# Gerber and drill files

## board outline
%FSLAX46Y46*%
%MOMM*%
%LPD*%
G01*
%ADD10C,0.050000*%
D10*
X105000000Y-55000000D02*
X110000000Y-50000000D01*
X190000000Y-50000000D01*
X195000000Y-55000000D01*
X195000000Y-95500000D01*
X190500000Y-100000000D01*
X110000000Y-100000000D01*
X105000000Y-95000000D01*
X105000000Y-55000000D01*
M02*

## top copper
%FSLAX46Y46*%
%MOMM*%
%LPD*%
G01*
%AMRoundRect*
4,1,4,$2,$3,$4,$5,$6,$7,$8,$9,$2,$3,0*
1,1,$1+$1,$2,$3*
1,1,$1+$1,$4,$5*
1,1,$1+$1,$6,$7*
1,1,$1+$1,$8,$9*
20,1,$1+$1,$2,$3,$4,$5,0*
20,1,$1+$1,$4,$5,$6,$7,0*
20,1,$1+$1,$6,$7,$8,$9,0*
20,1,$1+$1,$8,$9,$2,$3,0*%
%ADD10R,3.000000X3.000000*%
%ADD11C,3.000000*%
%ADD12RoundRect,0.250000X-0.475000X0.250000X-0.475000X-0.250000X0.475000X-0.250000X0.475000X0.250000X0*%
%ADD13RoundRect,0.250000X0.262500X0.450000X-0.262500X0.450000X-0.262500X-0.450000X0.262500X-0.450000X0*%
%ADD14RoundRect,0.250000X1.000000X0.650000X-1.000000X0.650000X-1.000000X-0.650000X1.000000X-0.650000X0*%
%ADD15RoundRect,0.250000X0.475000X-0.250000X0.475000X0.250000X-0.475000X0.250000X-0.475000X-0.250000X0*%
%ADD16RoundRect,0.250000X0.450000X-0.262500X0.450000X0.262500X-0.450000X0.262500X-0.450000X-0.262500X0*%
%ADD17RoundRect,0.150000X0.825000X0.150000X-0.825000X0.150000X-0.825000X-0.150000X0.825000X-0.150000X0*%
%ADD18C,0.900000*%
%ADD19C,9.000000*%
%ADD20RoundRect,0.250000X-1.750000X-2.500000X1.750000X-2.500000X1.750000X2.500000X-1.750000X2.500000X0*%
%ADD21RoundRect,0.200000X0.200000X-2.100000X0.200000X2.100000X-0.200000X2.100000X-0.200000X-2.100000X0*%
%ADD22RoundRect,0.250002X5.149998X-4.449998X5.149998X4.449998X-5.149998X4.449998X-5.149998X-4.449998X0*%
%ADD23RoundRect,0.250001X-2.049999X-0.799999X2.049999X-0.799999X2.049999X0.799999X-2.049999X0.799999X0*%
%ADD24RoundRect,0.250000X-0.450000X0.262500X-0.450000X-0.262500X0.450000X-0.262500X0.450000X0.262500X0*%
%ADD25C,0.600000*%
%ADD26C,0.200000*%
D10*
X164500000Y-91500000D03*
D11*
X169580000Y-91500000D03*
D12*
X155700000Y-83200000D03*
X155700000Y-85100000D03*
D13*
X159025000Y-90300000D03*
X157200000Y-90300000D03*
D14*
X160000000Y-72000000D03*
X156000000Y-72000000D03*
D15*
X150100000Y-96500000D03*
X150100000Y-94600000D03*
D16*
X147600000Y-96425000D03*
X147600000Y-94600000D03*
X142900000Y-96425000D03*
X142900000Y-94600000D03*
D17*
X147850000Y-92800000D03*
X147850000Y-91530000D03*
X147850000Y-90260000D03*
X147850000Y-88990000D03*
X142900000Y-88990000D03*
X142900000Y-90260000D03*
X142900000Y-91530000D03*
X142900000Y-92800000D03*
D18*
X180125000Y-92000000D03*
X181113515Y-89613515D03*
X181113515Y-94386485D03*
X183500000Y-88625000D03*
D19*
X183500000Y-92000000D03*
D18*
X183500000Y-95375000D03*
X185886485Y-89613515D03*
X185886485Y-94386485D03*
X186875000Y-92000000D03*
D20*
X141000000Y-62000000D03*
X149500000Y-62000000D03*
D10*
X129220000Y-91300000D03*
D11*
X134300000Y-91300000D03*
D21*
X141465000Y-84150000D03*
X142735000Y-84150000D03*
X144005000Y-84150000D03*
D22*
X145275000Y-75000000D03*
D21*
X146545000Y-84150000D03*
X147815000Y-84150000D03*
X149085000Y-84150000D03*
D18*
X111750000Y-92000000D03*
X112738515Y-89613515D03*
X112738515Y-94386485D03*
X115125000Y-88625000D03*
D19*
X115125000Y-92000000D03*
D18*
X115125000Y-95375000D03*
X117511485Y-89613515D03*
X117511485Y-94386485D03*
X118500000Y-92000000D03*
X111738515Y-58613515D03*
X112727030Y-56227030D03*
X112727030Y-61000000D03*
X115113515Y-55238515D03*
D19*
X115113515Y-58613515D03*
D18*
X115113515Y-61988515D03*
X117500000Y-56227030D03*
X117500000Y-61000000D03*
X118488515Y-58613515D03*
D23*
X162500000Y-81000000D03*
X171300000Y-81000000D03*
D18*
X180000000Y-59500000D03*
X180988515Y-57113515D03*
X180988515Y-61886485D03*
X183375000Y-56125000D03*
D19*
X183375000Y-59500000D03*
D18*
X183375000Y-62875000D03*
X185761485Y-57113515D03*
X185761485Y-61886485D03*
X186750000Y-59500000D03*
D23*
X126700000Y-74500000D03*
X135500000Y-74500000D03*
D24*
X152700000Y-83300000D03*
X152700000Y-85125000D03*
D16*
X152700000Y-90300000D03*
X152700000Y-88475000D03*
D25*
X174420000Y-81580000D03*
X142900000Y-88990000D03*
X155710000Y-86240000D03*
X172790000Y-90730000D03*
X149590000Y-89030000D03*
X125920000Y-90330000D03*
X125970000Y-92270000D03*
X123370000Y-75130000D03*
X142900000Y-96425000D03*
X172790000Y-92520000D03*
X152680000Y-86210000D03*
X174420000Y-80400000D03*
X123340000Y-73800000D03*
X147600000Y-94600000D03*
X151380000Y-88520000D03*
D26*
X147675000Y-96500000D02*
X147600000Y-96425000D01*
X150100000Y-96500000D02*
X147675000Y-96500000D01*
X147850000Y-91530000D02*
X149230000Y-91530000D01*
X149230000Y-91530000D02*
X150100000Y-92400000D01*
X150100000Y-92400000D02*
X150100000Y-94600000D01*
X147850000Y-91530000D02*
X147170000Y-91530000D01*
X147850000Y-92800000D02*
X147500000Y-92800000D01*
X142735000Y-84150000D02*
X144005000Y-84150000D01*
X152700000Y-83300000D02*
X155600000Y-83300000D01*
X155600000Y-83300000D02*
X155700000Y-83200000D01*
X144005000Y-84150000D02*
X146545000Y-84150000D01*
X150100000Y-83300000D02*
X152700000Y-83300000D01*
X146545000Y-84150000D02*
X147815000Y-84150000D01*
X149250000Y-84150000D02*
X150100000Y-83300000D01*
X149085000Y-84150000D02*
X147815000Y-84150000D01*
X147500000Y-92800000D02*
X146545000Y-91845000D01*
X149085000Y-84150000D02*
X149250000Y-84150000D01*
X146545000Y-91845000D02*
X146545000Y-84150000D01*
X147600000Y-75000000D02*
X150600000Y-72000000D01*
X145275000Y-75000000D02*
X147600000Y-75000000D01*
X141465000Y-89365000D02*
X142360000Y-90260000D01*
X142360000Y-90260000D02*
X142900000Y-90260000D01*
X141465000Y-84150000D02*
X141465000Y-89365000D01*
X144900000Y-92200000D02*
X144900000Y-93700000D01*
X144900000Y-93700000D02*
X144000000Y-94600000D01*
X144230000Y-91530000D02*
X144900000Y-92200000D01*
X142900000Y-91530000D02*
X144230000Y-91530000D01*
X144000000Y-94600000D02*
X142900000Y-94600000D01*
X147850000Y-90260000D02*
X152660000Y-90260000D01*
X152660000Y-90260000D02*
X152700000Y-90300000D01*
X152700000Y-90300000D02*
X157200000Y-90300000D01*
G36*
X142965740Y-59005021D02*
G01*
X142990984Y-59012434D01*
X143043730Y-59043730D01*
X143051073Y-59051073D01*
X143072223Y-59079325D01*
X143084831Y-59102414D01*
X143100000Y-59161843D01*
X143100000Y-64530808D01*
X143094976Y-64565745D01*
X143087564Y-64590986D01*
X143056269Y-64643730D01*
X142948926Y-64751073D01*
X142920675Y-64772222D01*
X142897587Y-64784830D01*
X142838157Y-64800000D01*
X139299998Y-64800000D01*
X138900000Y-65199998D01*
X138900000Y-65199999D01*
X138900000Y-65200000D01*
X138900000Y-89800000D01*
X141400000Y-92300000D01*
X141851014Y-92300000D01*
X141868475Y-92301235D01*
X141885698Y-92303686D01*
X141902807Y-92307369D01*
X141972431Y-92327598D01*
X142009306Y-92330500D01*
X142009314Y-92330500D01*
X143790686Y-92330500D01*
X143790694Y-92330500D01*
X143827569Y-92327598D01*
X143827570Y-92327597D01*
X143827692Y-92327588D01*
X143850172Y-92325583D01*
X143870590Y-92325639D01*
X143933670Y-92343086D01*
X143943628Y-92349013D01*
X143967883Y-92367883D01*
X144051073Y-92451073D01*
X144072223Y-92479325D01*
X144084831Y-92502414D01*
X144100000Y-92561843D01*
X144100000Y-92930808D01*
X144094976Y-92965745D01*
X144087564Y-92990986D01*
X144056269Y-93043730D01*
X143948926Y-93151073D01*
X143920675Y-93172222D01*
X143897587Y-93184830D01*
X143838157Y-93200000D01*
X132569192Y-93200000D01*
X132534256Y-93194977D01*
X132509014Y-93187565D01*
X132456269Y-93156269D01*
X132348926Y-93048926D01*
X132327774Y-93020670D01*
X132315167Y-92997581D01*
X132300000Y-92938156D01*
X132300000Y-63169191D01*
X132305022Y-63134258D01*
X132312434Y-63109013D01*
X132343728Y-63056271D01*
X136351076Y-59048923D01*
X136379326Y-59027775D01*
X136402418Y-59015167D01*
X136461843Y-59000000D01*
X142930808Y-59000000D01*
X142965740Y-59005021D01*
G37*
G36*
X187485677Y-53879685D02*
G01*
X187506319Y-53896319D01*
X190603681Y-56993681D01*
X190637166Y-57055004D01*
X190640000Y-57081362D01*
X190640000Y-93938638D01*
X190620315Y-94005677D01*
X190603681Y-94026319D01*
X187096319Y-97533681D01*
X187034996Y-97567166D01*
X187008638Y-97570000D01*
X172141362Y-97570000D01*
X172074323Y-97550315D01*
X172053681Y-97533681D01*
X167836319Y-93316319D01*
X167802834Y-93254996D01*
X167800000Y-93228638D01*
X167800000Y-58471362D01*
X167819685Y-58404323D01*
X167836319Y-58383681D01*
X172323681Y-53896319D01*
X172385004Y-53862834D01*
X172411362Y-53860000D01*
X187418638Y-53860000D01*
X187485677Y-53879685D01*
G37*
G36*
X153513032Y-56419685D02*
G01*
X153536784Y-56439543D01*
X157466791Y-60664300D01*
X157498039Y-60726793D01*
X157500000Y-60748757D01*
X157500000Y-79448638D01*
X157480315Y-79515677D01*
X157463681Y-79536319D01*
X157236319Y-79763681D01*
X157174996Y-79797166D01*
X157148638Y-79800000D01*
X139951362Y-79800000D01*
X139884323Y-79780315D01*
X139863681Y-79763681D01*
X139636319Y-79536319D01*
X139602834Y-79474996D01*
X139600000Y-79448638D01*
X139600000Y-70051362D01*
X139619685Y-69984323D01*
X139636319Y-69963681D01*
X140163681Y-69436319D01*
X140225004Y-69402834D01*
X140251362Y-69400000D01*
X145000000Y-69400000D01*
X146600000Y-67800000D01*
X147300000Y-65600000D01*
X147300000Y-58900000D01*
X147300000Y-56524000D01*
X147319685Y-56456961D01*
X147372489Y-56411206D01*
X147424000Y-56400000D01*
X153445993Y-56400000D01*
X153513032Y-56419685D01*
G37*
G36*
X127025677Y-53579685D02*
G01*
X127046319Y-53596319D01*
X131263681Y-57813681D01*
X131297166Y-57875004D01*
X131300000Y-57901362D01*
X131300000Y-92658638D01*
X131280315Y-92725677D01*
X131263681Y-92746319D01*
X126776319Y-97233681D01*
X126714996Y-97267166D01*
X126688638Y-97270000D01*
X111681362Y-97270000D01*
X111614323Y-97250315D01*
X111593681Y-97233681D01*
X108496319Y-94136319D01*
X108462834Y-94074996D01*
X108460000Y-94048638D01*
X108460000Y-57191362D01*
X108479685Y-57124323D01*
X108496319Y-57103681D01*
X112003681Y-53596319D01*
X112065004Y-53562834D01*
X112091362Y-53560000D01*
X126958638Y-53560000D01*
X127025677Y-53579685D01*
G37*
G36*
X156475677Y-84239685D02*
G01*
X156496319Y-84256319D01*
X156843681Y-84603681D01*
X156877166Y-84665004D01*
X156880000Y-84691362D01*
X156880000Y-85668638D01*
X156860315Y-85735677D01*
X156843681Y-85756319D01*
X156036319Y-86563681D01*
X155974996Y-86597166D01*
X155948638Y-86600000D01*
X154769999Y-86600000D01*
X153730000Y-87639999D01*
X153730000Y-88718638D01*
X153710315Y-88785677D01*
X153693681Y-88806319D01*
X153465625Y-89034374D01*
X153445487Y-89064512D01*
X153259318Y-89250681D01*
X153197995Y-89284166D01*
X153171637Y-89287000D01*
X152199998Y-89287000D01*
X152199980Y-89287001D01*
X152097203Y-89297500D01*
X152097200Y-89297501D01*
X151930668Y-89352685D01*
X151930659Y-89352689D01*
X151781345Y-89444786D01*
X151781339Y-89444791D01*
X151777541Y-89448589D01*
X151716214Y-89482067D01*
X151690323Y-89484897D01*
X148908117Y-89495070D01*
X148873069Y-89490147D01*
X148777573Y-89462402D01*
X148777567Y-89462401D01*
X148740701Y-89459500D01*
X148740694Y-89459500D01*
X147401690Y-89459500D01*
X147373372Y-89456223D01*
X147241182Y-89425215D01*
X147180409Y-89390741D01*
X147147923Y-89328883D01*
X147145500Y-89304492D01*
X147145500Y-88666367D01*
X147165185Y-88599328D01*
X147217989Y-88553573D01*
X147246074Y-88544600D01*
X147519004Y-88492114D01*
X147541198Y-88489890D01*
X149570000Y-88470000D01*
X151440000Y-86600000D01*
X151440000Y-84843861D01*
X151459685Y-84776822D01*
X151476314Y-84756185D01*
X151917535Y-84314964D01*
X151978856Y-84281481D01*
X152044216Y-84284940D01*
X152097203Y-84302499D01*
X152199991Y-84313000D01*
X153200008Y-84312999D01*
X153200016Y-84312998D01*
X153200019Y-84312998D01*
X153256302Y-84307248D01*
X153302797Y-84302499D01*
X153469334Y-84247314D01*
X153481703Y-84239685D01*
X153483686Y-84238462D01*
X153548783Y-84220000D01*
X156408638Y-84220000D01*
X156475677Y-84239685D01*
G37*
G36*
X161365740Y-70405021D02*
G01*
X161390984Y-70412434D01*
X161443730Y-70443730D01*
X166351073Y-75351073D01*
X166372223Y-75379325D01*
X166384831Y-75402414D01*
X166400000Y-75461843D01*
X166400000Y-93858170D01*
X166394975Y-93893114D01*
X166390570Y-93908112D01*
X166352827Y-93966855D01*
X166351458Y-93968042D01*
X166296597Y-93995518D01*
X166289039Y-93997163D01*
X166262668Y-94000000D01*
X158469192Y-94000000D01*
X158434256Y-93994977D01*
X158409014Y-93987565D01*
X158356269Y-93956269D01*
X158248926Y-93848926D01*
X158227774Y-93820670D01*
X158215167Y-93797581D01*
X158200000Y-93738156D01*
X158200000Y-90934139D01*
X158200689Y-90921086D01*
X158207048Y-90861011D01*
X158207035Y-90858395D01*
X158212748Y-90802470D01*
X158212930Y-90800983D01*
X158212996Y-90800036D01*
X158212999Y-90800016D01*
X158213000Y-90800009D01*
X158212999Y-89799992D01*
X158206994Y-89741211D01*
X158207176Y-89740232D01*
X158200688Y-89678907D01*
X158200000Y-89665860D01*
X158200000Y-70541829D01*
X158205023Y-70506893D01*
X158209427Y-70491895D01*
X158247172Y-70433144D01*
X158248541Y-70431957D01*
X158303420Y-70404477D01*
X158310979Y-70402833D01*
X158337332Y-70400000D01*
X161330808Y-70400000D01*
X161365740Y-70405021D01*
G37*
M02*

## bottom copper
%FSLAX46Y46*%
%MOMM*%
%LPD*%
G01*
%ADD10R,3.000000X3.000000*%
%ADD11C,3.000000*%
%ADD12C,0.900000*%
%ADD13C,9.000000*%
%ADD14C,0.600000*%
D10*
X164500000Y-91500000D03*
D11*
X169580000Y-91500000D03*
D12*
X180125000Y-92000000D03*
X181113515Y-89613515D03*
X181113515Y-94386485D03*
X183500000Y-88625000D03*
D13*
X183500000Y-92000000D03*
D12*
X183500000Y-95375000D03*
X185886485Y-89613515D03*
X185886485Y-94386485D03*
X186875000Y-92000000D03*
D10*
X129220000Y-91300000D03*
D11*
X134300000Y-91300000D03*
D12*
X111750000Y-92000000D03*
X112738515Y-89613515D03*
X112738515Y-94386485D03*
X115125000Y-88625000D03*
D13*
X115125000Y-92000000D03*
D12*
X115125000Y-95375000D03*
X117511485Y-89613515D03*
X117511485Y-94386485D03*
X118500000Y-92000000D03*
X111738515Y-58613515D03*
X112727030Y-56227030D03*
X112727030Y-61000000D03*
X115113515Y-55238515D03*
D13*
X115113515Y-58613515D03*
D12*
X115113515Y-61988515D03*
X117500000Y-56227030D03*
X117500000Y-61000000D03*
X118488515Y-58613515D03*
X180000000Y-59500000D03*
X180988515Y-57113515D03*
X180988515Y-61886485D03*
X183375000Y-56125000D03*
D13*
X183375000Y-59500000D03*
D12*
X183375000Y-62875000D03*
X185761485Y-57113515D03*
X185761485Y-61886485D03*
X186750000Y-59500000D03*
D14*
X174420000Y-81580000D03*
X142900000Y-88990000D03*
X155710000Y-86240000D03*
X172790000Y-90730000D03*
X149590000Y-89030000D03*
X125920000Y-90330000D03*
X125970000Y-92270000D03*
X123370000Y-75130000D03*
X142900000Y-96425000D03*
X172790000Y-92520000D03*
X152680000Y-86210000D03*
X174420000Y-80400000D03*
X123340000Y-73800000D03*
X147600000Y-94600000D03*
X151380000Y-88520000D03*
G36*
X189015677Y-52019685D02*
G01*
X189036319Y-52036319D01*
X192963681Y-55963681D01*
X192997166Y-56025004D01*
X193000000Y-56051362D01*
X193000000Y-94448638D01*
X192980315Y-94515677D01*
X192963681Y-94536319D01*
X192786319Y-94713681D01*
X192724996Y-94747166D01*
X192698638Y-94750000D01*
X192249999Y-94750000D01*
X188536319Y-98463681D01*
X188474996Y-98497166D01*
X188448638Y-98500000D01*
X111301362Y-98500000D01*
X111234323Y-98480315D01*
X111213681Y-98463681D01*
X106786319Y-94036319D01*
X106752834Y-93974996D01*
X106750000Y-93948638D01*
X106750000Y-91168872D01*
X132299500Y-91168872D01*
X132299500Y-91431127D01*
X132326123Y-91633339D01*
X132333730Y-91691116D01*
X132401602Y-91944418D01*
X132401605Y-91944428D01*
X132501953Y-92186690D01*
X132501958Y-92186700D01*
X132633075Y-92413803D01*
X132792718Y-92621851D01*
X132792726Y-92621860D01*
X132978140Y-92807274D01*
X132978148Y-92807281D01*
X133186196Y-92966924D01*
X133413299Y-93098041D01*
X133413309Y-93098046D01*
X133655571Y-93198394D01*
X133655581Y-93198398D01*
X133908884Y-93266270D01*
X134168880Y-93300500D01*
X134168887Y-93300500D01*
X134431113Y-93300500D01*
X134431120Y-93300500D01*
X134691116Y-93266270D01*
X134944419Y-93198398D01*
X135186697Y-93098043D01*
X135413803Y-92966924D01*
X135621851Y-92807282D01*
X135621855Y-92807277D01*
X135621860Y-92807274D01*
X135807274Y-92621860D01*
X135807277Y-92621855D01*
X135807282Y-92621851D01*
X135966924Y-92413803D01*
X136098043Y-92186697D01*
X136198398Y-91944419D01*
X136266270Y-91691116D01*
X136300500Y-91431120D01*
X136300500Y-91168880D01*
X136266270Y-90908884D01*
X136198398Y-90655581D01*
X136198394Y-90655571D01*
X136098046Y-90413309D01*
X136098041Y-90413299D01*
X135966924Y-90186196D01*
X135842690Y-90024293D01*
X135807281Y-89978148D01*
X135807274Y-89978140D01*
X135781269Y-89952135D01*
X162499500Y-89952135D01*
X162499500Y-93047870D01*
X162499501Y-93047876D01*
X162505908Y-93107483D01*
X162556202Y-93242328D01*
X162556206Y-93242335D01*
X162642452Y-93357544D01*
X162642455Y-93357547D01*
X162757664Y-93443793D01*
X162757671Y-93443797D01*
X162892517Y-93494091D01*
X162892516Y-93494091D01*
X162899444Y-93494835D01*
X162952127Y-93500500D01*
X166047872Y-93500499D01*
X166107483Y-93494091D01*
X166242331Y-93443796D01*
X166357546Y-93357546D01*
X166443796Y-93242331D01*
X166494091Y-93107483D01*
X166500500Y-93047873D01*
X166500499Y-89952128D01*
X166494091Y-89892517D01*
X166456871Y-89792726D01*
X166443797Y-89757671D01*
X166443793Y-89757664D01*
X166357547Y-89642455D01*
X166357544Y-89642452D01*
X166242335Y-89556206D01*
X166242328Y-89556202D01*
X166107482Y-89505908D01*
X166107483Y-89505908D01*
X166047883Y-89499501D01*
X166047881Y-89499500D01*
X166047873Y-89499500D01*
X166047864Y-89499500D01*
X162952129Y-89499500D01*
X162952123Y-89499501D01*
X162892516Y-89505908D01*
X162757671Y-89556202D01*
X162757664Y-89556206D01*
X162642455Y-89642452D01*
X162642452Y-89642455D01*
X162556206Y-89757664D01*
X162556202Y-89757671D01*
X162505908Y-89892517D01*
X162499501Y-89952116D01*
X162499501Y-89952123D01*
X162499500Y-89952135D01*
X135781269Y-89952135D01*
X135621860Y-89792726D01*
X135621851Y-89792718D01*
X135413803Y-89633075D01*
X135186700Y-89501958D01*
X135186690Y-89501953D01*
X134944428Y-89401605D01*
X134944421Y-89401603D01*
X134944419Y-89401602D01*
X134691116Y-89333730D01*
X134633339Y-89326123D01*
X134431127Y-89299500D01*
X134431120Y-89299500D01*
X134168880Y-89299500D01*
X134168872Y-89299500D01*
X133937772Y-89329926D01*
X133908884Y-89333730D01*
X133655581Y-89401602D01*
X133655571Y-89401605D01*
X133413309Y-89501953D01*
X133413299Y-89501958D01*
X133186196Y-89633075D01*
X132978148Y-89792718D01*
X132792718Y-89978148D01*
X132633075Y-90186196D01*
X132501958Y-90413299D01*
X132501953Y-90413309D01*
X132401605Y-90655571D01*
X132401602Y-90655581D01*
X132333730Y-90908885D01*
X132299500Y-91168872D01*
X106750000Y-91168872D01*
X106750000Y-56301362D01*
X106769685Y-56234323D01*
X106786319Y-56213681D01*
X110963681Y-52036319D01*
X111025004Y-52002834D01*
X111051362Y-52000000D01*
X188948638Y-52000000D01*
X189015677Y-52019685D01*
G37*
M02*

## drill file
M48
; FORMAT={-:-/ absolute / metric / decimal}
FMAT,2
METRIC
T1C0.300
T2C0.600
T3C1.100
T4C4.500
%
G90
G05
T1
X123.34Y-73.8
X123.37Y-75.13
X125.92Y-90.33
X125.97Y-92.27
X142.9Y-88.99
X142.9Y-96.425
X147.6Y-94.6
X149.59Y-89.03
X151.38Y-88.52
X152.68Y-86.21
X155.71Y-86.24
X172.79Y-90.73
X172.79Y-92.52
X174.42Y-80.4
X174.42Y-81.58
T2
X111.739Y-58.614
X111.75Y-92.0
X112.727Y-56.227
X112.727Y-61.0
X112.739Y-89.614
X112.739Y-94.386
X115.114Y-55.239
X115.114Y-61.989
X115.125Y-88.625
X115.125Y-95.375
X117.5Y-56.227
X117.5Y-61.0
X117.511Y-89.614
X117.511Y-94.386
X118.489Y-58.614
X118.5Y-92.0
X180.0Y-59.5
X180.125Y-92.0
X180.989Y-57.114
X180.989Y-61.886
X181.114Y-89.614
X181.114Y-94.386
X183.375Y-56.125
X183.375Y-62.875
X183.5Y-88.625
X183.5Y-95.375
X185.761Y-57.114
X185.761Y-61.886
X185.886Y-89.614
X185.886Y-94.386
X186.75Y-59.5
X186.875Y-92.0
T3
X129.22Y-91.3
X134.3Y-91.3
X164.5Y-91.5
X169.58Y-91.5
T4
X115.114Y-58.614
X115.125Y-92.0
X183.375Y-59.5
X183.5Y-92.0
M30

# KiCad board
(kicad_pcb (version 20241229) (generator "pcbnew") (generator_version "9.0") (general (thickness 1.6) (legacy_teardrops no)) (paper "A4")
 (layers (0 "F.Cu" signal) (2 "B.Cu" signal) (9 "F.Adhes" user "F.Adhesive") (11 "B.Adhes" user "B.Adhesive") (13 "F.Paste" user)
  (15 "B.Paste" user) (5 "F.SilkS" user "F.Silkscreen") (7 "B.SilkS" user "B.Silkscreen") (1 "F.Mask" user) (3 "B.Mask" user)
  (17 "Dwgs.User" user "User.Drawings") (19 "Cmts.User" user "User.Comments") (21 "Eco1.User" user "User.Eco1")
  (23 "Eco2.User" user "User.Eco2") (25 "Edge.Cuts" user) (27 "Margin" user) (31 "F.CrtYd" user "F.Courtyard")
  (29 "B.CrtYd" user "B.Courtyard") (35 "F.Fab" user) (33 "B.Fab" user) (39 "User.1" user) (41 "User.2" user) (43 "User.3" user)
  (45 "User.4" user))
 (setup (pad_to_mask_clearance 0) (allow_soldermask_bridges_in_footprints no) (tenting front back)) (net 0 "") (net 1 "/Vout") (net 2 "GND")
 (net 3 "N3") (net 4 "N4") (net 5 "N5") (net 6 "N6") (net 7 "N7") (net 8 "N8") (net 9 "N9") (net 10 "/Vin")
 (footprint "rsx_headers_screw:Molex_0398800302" (layer "F.Cu") (at 164.5 91.5)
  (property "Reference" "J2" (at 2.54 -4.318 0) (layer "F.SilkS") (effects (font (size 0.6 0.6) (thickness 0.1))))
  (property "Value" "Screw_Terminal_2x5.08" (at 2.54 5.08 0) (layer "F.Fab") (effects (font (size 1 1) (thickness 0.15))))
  (pad "1" thru_hole rect (at 0 0) (size 3 3) (drill 1.1) (layers "*.Cu" "*.Mask") (remove_unused_layers no) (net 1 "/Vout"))
  (pad "2" thru_hole circle (at 5.08 0) (size 3 3) (drill 1.1) (layers "*.Cu" "*.Mask") (remove_unused_layers no) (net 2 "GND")))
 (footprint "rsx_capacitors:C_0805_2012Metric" (layer "F.Cu") (at 155.7 84.15 -90)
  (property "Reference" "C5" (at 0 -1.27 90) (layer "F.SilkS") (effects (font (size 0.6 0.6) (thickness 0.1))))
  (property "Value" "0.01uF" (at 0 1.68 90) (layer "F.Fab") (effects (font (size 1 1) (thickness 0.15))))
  (pad "1" smd roundrect (at -0.95 0 270) (size 1 1.45) (layers "F.Cu" "F.Mask" "F.Paste") (roundrect_rratio 0.25) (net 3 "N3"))
  (pad "2" smd roundrect (at 0.95 0 270) (size 1 1.45) (layers "F.Cu" "F.Mask" "F.Paste") (roundrect_rratio 0.25) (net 2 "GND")))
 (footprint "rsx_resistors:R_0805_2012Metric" (layer "F.Cu") (at 158.1125 90.3 180)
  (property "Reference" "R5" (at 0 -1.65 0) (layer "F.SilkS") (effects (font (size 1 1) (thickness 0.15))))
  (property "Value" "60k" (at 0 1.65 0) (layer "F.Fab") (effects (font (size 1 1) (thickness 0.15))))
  (pad "1" smd roundrect (at -0.9125 0 180) (size 1.025 1.4) (layers "F.Cu" "F.Mask" "F.Paste") (roundrect_rratio 0.243902) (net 1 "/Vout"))
  (pad "2" smd roundrect (at 0.9125 0 180) (size 1.025 1.4) (layers "F.Cu" "F.Mask" "F.Paste") (roundrect_rratio 0.243902) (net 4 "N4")))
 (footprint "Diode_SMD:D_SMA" (layer "F.Cu") (at 158 72 180)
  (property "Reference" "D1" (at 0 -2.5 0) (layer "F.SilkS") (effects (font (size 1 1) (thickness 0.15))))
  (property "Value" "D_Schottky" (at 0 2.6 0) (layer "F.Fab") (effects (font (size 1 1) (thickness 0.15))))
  (pad "1" smd roundrect (at -2 0 180) (size 2.5 1.8) (layers "F.Cu" "F.Mask" "F.Paste") (roundrect_rratio 0.1388888889) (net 1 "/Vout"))
  (pad "2" smd roundrect (at 2 0 180) (size 2.5 1.8) (layers "F.Cu" "F.Mask" "F.Paste") (roundrect_rratio 0.1388888889) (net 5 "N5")))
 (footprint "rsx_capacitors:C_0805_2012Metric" (layer "F.Cu") (at 150.1 95.55 90)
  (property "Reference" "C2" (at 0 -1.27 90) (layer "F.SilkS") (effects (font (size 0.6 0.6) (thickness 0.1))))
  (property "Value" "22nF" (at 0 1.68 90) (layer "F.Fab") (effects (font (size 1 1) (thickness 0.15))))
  (pad "1" smd roundrect (at -0.95 0 90) (size 1 1.45) (layers "F.Cu" "F.Mask" "F.Paste") (roundrect_rratio 0.25) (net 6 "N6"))
  (pad "2" smd roundrect (at 0.95 0 90) (size 1 1.45) (layers "F.Cu" "F.Mask" "F.Paste") (roundrect_rratio 0.25) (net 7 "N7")))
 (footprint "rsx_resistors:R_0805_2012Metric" (layer "F.Cu") (at 147.6 95.5125 90)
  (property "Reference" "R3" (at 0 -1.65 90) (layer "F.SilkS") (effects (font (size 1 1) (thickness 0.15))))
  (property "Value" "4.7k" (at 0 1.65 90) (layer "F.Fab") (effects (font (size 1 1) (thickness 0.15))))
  (pad "1" smd roundrect (at -0.9125 0 90) (size 1.025 1.4) (layers "F.Cu" "F.Mask" "F.Paste") (roundrect_rratio 0.243902) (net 6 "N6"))
  (pad "2" smd roundrect (at 0.9125 0 90) (size 1.025 1.4) (layers "F.Cu" "F.Mask" "F.Paste") (roundrect_rratio 0.243902) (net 2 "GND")))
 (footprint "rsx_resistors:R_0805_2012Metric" (layer "F.Cu") (at 142.9 95.5125 90)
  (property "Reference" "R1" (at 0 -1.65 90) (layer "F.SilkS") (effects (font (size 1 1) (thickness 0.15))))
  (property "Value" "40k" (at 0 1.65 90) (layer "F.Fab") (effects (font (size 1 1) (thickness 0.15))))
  (pad "1" smd roundrect (at -0.9125 0 90) (size 1.025 1.4) (layers "F.Cu" "F.Mask" "F.Paste") (roundrect_rratio 0.243902) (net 2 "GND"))
  (pad "2" smd roundrect (at 0.9125 0 90) (size 1.025 1.4) (layers "F.Cu" "F.Mask" "F.Paste") (roundrect_rratio 0.243902) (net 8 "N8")))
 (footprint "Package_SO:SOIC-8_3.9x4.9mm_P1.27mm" (layer "F.Cu") (at 145.375 90.895 180)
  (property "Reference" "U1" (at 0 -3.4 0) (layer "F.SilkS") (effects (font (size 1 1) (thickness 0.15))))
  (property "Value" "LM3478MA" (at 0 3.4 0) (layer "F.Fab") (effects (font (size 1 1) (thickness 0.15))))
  (pad "1" smd roundrect (at -2.475 -1.905 180) (size 1.95 0.6) (layers "F.Cu" "F.Mask" "F.Paste") (roundrect_rratio 0.25) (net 3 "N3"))
  (pad "2" smd roundrect (at -2.475 -0.635 180) (size 1.95 0.6) (layers "F.Cu" "F.Mask" "F.Paste") (roundrect_rratio 0.25) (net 7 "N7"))
  (pad "3" smd roundrect (at -2.475 0.635 180) (size 1.95 0.6) (layers "F.Cu" "F.Mask" "F.Paste") (roundrect_rratio 0.25) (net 4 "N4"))
  (pad "4" smd roundrect (at -2.475 1.905 180) (size 1.95 0.6) (layers "F.Cu" "F.Mask" "F.Paste") (roundrect_rratio 0.25) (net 2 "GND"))
  (pad "5" smd roundrect (at 2.475 1.905 180) (size 1.95 0.6) (layers "F.Cu" "F.Mask" "F.Paste") (roundrect_rratio 0.25) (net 2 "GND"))
  (pad "6" smd roundrect (at 2.475 0.635 180) (size 1.95 0.6) (layers "F.Cu" "F.Mask" "F.Paste") (roundrect_rratio 0.25) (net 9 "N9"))
  (pad "7" smd roundrect (at 2.475 -0.635 180) (size 1.95 0.6) (layers "F.Cu" "F.Mask" "F.Paste") (roundrect_rratio 0.25) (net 8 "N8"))
  (pad "8" smd roundrect (at 2.475 -1.905 180) (size 1.95 0.6) (layers "F.Cu" "F.Mask" "F.Paste") (roundrect_rratio 0.25) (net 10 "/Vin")))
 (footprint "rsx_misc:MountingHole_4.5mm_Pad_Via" (layer "F.Cu") (at 183.5 92)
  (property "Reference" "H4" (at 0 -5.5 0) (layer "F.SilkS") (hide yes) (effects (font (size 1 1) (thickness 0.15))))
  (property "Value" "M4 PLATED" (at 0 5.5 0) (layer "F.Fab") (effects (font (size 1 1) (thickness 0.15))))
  (pad "1" thru_hole circle (at -3.375 0) (size 0.9 0.9) (drill 0.6) (layers "*.Cu" "*.Mask") (remove_unused_layers no) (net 2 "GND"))
  (pad "1" thru_hole circle (at -2.386485 -2.386485) (size 0.9 0.9) (drill 0.6) (layers "*.Cu" "*.Mask") (remove_unused_layers no)
   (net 2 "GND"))
  (pad "1" thru_hole circle (at -2.386485 2.386485) (size 0.9 0.9) (drill 0.6) (layers "*.Cu" "*.Mask") (remove_unused_layers no)
   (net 2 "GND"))
  (pad "1" thru_hole circle (at 0 -3.375) (size 0.9 0.9) (drill 0.6) (layers "*.Cu" "*.Mask") (remove_unused_layers no) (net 2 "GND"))
  (pad "1" thru_hole circle (at 0 0) (size 9 9) (drill 4.5) (layers "*.Cu" "*.Mask") (remove_unused_layers no) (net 2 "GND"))
  (pad "1" thru_hole circle (at 0 3.375) (size 0.9 0.9) (drill 0.6) (layers "*.Cu" "*.Mask") (remove_unused_layers no) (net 2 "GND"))
  (pad "1" thru_hole circle (at 2.386485 -2.386485) (size 0.9 0.9) (drill 0.6) (layers "*.Cu" "*.Mask") (remove_unused_layers no)
   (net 2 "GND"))
  (pad "1" thru_hole circle (at 2.386485 2.386485) (size 0.9 0.9) (drill 0.6) (layers "*.Cu" "*.Mask") (remove_unused_layers no)
   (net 2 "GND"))
  (pad "1" thru_hole circle (at 3.375 0) (size 0.9 0.9) (drill 0.6) (layers "*.Cu" "*.Mask") (remove_unused_layers no) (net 2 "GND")))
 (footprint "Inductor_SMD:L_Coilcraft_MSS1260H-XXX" (layer "F.Cu") (at 145.25 62)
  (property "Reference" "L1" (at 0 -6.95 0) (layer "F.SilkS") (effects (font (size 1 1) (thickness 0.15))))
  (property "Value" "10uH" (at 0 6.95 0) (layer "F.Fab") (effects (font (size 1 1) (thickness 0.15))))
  (pad "1" smd roundrect (at -4.25 0) (size 4 5.5) (layers "F.Cu" "F.Mask" "F.Paste") (roundrect_rratio 0.0625) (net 10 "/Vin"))
  (pad "2" smd roundrect (at 4.25 0) (size 4 5.5) (layers "F.Cu" "F.Mask" "F.Paste") (roundrect_rratio 0.0625) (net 5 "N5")))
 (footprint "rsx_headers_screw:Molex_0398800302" (layer "F.Cu") (at 129.22 91.3)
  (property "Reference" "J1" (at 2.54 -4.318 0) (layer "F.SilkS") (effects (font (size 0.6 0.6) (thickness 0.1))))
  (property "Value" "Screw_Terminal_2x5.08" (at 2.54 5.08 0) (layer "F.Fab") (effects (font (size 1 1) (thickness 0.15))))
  (pad "1" thru_hole rect (at 0 0) (size 3 3) (drill 1.1) (layers "*.Cu" "*.Mask") (remove_unused_layers no) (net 2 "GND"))
  (pad "2" thru_hole circle (at 5.08 0) (size 3 3) (drill 1.1) (layers "*.Cu" "*.Mask") (remove_unused_layers no) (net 10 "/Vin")))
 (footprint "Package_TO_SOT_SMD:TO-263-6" (layer "F.Cu") (at 145.275 76.5 90)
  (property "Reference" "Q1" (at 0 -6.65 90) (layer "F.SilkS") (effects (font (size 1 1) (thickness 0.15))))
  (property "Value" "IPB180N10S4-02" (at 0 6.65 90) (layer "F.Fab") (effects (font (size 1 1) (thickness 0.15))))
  (pad "" smd roundrect (at -0.925 -2.775 90) (size 4.55 5.25) (layers "F.Paste") (roundrect_rratio 0.054945))
  (pad "" smd roundrect (at -0.925 2.775 90) (size 4.55 5.25) (layers "F.Paste") (roundrect_rratio 0.054945))
  (pad "" smd roundrect (at 3.925 -2.775 90) (size 4.55 5.25) (layers "F.Paste") (roundrect_rratio 0.054945))
  (pad "" smd roundrect (at 3.925 2.775 90) (size 4.55 5.25) (layers "F.Paste") (roundrect_rratio 0.054945))
  (pad "1" smd roundrect (at -7.65 -3.81 90) (size 4.6 0.8) (layers "F.Cu" "F.Mask" "F.Paste") (roundrect_rratio 0.25) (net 9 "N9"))
  (pad "2" smd roundrect (at -7.65 -2.54 90) (size 4.6 0.8) (layers "F.Cu" "F.Mask" "F.Paste") (roundrect_rratio 0.25) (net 3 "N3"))
  (pad "3" smd roundrect (at -7.65 -1.27 90) (size 4.6 0.8) (layers "F.Cu" "F.Mask" "F.Paste") (roundrect_rratio 0.25) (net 3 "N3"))
  (pad "4" smd roundrect (at 1.5 0 90) (size 9.4 10.8) (layers "F.Cu" "F.Mask") (roundrect_rratio 0.026596) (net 5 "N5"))
  (pad "5" smd roundrect (at -7.65 1.27 90) (size 4.6 0.8) (layers "F.Cu" "F.Mask" "F.Paste") (roundrect_rratio 0.25) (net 3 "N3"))
  (pad "6" smd roundrect (at -7.65 2.54 90) (size 4.6 0.8) (layers "F.Cu" "F.Mask" "F.Paste") (roundrect_rratio 0.25) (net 3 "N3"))
  (pad "7" smd roundrect (at -7.65 3.81 90) (size 4.6 0.8) (layers "F.Cu" "F.Mask" "F.Paste") (roundrect_rratio 0.25) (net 3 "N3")))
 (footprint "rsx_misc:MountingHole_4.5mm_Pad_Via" (layer "F.Cu") (at 115.125 92)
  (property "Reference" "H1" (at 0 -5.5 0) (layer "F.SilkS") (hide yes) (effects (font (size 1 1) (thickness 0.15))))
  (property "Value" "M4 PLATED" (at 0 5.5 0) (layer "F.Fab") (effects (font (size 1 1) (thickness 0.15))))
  (pad "1" thru_hole circle (at -3.375 0) (size 0.9 0.9) (drill 0.6) (layers "*.Cu" "*.Mask") (remove_unused_layers no) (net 2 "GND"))
  (pad "1" thru_hole circle (at -2.386485 -2.386485) (size 0.9 0.9) (drill 0.6) (layers "*.Cu" "*.Mask") (remove_unused_layers no)
   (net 2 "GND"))
  (pad "1" thru_hole circle (at -2.386485 2.386485) (size 0.9 0.9) (drill 0.6) (layers "*.Cu" "*.Mask") (remove_unused_layers no)
   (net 2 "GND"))
  (pad "1" thru_hole circle (at 0 -3.375) (size 0.9 0.9) (drill 0.6) (layers "*.Cu" "*.Mask") (remove_unused_layers no) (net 2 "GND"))
  (pad "1" thru_hole circle (at 0 0) (size 9 9) (drill 4.5) (layers "*.Cu" "*.Mask") (remove_unused_layers no) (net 2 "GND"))
  (pad "1" thru_hole circle (at 0 3.375) (size 0.9 0.9) (drill 0.6) (layers "*.Cu" "*.Mask") (remove_unused_layers no) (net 2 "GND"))
  (pad "1" thru_hole circle (at 2.386485 -2.386485) (size 0.9 0.9) (drill 0.6) (layers "*.Cu" "*.Mask") (remove_unused_layers no)
   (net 2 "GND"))
  (pad "1" thru_hole circle (at 2.386485 2.386485) (size 0.9 0.9) (drill 0.6) (layers "*.Cu" "*.Mask") (remove_unused_layers no)
   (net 2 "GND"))
  (pad "1" thru_hole circle (at 3.375 0) (size 0.9 0.9) (drill 0.6) (layers "*.Cu" "*.Mask") (remove_unused_layers no) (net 2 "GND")))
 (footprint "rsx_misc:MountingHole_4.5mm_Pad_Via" (layer "F.Cu") (at 115.113515 58.613515)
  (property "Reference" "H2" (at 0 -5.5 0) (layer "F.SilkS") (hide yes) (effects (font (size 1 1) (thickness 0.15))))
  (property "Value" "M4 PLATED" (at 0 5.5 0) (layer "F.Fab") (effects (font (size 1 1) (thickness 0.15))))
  (pad "1" thru_hole circle (at -3.375 0) (size 0.9 0.9) (drill 0.6) (layers "*.Cu" "*.Mask") (remove_unused_layers no) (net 2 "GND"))
  (pad "1" thru_hole circle (at -2.386485 -2.386485) (size 0.9 0.9) (drill 0.6) (layers "*.Cu" "*.Mask") (remove_unused_layers no)
   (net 2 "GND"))
  (pad "1" thru_hole circle (at -2.386485 2.386485) (size 0.9 0.9) (drill 0.6) (layers "*.Cu" "*.Mask") (remove_unused_layers no)
   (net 2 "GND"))
  (pad "1" thru_hole circle (at 0 -3.375) (size 0.9 0.9) (drill 0.6) (layers "*.Cu" "*.Mask") (remove_unused_layers no) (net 2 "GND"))
  (pad "1" thru_hole circle (at 0 0) (size 9 9) (drill 4.5) (layers "*.Cu" "*.Mask") (remove_unused_layers no) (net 2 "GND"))
  (pad "1" thru_hole circle (at 0 3.375) (size 0.9 0.9) (drill 0.6) (layers "*.Cu" "*.Mask") (remove_unused_layers no) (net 2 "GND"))
  (pad "1" thru_hole circle (at 2.386485 -2.386485) (size 0.9 0.9) (drill 0.6) (layers "*.Cu" "*.Mask") (remove_unused_layers no)
   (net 2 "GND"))
  (pad "1" thru_hole circle (at 2.386485 2.386485) (size 0.9 0.9) (drill 0.6) (layers "*.Cu" "*.Mask") (remove_unused_layers no)
   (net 2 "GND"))
  (pad "1" thru_hole circle (at 3.375 0) (size 0.9 0.9) (drill 0.6) (layers "*.Cu" "*.Mask") (remove_unused_layers no) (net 2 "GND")))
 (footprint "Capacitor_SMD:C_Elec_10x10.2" (layer "F.Cu") (at 166.9 81)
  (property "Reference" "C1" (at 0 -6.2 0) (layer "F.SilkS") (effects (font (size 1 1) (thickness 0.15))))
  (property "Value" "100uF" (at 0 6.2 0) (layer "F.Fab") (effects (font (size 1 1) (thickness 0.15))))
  (pad "1" smd roundrect (at -4.4 0) (size 4.6 2.1) (layers "F.Cu" "F.Mask" "F.Paste") (roundrect_rratio 0.119048) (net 1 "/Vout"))
  (pad "2" smd roundrect (at 4.4 0) (size 4.6 2.1) (layers "F.Cu" "F.Mask" "F.Paste") (roundrect_rratio 0.119048) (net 2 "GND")))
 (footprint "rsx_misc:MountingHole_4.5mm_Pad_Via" (layer "F.Cu") (at 183.375 59.5)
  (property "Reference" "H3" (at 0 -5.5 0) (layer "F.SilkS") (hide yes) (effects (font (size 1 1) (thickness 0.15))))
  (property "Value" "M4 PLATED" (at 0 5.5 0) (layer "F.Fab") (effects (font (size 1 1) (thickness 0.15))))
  (pad "1" thru_hole circle (at -3.375 0) (size 0.9 0.9) (drill 0.6) (layers "*.Cu" "*.Mask") (remove_unused_layers no) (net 2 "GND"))
  (pad "1" thru_hole circle (at -2.386485 -2.386485) (size 0.9 0.9) (drill 0.6) (layers "*.Cu" "*.Mask") (remove_unused_layers no)
   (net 2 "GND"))
  (pad "1" thru_hole circle (at -2.386485 2.386485) (size 0.9 0.9) (drill 0.6) (layers "*.Cu" "*.Mask") (remove_unused_layers no)
   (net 2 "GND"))
  (pad "1" thru_hole circle (at 0 -3.375) (size 0.9 0.9) (drill 0.6) (layers "*.Cu" "*.Mask") (remove_unused_layers no) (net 2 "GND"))
  (pad "1" thru_hole circle (at 0 0) (size 9 9) (drill 4.5) (layers "*.Cu" "*.Mask") (remove_unused_layers no) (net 2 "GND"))
  (pad "1" thru_hole circle (at 0 3.375) (size 0.9 0.9) (drill 0.6) (layers "*.Cu" "*.Mask") (remove_unused_layers no) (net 2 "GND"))
  (pad "1" thru_hole circle (at 2.386485 -2.386485) (size 0.9 0.9) (drill 0.6) (layers "*.Cu" "*.Mask") (remove_unused_layers no)
   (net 2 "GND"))
  (pad "1" thru_hole circle (at 2.386485 2.386485) (size 0.9 0.9) (drill 0.6) (layers "*.Cu" "*.Mask") (remove_unused_layers no)
   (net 2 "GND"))
  (pad "1" thru_hole circle (at 3.375 0) (size 0.9 0.9) (drill 0.6) (layers "*.Cu" "*.Mask") (remove_unused_layers no) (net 2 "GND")))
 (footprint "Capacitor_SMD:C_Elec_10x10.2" (layer "F.Cu") (at 131.1 74.5)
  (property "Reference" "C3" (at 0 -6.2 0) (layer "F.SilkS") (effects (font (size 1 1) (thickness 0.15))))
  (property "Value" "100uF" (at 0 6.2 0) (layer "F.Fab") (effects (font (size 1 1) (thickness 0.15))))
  (pad "1" smd roundrect (at -4.4 0) (size 4.6 2.1) (layers "F.Cu" "F.Mask" "F.Paste") (roundrect_rratio 0.119048) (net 2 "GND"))
  (pad "2" smd roundrect (at 4.4 0) (size 4.6 2.1) (layers "F.Cu" "F.Mask" "F.Paste") (roundrect_rratio 0.119048) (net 10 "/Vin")))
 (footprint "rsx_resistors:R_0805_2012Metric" (layer "F.Cu") (at 152.7 84.2125 -90)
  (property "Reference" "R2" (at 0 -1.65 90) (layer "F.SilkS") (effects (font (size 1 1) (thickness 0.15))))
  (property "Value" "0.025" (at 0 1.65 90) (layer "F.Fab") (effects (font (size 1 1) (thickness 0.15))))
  (pad "1" smd roundrect (at -0.9125 0 270) (size 1.025 1.4) (layers "F.Cu" "F.Mask" "F.Paste") (roundrect_rratio 0.243902) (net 3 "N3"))
  (pad "2" smd roundrect (at 0.9125 0 270) (size 1.025 1.4) (layers "F.Cu" "F.Mask" "F.Paste") (roundrect_rratio 0.243902) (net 2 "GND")))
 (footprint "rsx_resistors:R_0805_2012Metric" (layer "F.Cu") (at 152.7 89.3875 90)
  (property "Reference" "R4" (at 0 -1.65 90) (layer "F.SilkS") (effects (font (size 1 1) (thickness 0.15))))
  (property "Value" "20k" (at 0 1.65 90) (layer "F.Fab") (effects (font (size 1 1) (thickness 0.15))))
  (pad "1" smd roundrect (at -0.9125 0 90) (size 1.025 1.4) (layers "F.Cu" "F.Mask" "F.Paste") (roundrect_rratio 0.243902) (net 4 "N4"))
  (pad "2" smd roundrect (at 0.9125 0 90) (size 1.025 1.4) (layers "F.Cu" "F.Mask" "F.Paste") (roundrect_rratio 0.243902) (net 2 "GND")))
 (gr_poly
  (pts (xy 105 55) (xy 110 50) (xy 190 50) (xy 195 55) (xy 195 95.5) (xy 190.5 100) (xy 110 100) (xy 105 95))
  (stroke (width 0.05) (type solid)) (fill no) (layer "Edge.Cuts"))
 (via (at 174.42 81.58) (size 0.6) (drill 0.3) (layers "F.Cu" "B.Cu") (free yes) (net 2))
 (via (at 142.9 88.99) (size 0.6) (drill 0.3) (layers "F.Cu" "B.Cu") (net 2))
 (via (at 155.71 86.24) (size 0.6) (drill 0.3) (layers "F.Cu" "B.Cu") (free yes) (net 2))
 (via (at 172.79 90.73) (size 0.6) (drill 0.3) (layers "F.Cu" "B.Cu") (free yes) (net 2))
 (via (at 149.59 89.03) (size 0.6) (drill 0.3) (layers "F.Cu" "B.Cu") (free yes) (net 2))
 (via (at 125.92 90.33) (size 0.6) (drill 0.3) (layers "F.Cu" "B.Cu") (free yes) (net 2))
 (via (at 125.97 92.27) (size 0.6) (drill 0.3) (layers "F.Cu" "B.Cu") (free yes) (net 2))
 (via (at 123.37 75.13) (size 0.6) (drill 0.3) (layers "F.Cu" "B.Cu") (free yes) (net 2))
 (via (at 142.9 96.425) (size 0.6) (drill 0.3) (layers "F.Cu" "B.Cu") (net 2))
 (via (at 172.79 92.52) (size 0.6) (drill 0.3) (layers "F.Cu" "B.Cu") (free yes) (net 2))
 (via (at 152.68 86.21) (size 0.6) (drill 0.3) (layers "F.Cu" "B.Cu") (free yes) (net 2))
 (via (at 174.42 80.4) (size 0.6) (drill 0.3) (layers "F.Cu" "B.Cu") (free yes) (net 2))
 (via (at 123.34 73.8) (size 0.6) (drill 0.3) (layers "F.Cu" "B.Cu") (free yes) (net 2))
 (via (at 147.6 94.6) (size 0.6) (drill 0.3) (layers "F.Cu" "B.Cu") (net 2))
 (via (at 151.38 88.52) (size 0.6) (drill 0.3) (layers "F.Cu" "B.Cu") (free yes) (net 2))
 (segment (start 147.675 96.5) (end 147.6 96.425) (width 0.2) (layer "F.Cu") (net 6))
 (segment (start 150.1 96.5) (end 147.675 96.5) (width 0.2) (layer "F.Cu") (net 6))
 (segment (start 147.85 91.53) (end 149.23 91.53) (width 0.2) (layer "F.Cu") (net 7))
 (segment (start 149.23 91.53) (end 150.1 92.4) (width 0.2) (layer "F.Cu") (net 7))
 (segment (start 150.1 92.4) (end 150.1 94.6) (width 0.2) (layer "F.Cu") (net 7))
 (segment (start 147.85 91.53) (end 147.17 91.53) (width 0.2) (layer "F.Cu") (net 7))
 (segment (start 147.85 92.8) (end 147.5 92.8) (width 0.2) (layer "F.Cu") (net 3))
 (segment (start 142.735 84.15) (end 144.005 84.15) (width 0.2) (layer "F.Cu") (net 3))
 (segment (start 152.7 83.3) (end 155.6 83.3) (width 0.2) (layer "F.Cu") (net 3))
 (segment (start 155.6 83.3) (end 155.7 83.2) (width 0.2) (layer "F.Cu") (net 3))
 (segment (start 144.005 84.15) (end 146.545 84.15) (width 0.2) (layer "F.Cu") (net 3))
 (segment (start 150.1 83.3) (end 152.7 83.3) (width 0.2) (layer "F.Cu") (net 3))
 (segment (start 146.545 84.15) (end 147.815 84.15) (width 0.2) (layer "F.Cu") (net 3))
 (segment (start 149.25 84.15) (end 150.1 83.3) (width 0.2) (layer "F.Cu") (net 3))
 (segment (start 149.085 84.15) (end 147.815 84.15) (width 0.2) (layer "F.Cu") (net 3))
 (segment (start 147.5 92.8) (end 146.545 91.845) (width 0.2) (layer "F.Cu") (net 3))
 (segment (start 149.085 84.15) (end 149.25 84.15) (width 0.2) (layer "F.Cu") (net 3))
 (segment (start 146.545 91.845) (end 146.545 84.15) (width 0.2) (layer "F.Cu") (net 3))
 (segment (start 147.6 75) (end 150.6 72) (width 0.2) (layer "F.Cu") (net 5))
 (segment (start 145.275 75) (end 147.6 75) (width 0.2) (layer "F.Cu") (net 5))
 (segment (start 141.465 89.365) (end 142.36 90.26) (width 0.2) (layer "F.Cu") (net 9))
 (segment (start 142.36 90.26) (end 142.9 90.26) (width 0.2) (layer "F.Cu") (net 9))
 (segment (start 141.465 84.15) (end 141.465 89.365) (width 0.2) (layer "F.Cu") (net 9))
 (segment (start 144.9 92.2) (end 144.9 93.7) (width 0.2) (layer "F.Cu") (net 8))
 (segment (start 144.9 93.7) (end 144 94.6) (width 0.2) (layer "F.Cu") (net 8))
 (segment (start 144.23 91.53) (end 144.9 92.2) (width 0.2) (layer "F.Cu") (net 8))
 (segment (start 142.9 91.53) (end 144.23 91.53) (width 0.2) (layer "F.Cu") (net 8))
 (segment (start 144 94.6) (end 142.9 94.6) (width 0.2) (layer "F.Cu") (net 8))
 (segment (start 147.85 90.26) (end 152.66 90.26) (width 0.2) (layer "F.Cu") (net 4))
 (segment (start 152.66 90.26) (end 152.7 90.3) (width 0.2) (layer "F.Cu") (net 4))
 (segment (start 152.7 90.3) (end 157.2 90.3) (width 0.2) (layer "F.Cu") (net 4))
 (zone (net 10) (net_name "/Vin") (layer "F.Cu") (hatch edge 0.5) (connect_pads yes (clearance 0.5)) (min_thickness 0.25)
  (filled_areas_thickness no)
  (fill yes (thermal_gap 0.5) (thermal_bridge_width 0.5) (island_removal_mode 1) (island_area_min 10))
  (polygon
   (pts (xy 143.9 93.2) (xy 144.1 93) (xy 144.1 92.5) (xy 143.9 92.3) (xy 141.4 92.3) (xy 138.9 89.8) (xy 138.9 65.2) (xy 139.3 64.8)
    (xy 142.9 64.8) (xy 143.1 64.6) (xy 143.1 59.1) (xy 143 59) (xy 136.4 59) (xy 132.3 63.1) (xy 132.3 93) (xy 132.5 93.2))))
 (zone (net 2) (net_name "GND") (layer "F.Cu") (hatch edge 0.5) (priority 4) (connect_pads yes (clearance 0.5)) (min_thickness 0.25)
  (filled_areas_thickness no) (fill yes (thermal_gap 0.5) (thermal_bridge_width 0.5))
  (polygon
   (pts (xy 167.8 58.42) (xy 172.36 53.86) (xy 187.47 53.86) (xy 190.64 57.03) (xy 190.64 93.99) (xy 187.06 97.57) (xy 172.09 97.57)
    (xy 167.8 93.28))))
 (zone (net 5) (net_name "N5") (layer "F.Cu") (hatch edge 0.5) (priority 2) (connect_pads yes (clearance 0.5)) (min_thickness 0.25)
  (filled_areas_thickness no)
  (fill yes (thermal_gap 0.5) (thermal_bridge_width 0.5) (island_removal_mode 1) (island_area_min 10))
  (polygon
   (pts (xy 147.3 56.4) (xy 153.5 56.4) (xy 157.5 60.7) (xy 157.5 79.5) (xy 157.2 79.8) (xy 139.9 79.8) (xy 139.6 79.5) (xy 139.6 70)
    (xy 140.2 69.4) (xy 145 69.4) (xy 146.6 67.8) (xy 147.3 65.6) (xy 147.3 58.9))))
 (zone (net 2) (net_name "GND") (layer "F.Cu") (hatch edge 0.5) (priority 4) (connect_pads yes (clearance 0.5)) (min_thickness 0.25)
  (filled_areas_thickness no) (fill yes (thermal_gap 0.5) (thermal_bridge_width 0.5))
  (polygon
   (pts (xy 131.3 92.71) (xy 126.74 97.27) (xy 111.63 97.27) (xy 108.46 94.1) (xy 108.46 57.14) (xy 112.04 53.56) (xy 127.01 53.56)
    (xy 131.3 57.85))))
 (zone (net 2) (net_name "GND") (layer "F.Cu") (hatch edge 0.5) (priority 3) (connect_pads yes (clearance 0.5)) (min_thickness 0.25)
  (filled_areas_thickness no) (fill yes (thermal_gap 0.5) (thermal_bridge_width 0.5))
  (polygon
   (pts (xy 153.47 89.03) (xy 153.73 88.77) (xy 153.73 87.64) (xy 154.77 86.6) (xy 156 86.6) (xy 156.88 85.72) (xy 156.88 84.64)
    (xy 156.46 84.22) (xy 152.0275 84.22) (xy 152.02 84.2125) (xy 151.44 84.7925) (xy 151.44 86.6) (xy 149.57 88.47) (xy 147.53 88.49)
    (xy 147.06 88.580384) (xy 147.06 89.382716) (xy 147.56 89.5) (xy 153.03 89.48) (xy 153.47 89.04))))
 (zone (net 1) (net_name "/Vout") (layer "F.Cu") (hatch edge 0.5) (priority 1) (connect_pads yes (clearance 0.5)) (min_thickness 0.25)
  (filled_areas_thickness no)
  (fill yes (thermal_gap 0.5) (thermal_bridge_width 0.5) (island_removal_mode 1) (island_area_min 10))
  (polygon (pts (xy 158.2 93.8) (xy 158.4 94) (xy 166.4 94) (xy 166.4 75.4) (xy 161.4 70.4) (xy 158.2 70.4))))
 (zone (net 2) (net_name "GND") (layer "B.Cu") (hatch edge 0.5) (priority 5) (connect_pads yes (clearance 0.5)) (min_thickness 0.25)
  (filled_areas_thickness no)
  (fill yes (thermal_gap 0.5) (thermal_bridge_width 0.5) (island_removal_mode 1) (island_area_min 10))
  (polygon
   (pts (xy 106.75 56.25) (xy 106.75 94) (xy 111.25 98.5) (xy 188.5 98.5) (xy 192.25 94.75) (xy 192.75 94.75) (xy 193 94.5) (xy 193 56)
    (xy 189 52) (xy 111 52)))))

